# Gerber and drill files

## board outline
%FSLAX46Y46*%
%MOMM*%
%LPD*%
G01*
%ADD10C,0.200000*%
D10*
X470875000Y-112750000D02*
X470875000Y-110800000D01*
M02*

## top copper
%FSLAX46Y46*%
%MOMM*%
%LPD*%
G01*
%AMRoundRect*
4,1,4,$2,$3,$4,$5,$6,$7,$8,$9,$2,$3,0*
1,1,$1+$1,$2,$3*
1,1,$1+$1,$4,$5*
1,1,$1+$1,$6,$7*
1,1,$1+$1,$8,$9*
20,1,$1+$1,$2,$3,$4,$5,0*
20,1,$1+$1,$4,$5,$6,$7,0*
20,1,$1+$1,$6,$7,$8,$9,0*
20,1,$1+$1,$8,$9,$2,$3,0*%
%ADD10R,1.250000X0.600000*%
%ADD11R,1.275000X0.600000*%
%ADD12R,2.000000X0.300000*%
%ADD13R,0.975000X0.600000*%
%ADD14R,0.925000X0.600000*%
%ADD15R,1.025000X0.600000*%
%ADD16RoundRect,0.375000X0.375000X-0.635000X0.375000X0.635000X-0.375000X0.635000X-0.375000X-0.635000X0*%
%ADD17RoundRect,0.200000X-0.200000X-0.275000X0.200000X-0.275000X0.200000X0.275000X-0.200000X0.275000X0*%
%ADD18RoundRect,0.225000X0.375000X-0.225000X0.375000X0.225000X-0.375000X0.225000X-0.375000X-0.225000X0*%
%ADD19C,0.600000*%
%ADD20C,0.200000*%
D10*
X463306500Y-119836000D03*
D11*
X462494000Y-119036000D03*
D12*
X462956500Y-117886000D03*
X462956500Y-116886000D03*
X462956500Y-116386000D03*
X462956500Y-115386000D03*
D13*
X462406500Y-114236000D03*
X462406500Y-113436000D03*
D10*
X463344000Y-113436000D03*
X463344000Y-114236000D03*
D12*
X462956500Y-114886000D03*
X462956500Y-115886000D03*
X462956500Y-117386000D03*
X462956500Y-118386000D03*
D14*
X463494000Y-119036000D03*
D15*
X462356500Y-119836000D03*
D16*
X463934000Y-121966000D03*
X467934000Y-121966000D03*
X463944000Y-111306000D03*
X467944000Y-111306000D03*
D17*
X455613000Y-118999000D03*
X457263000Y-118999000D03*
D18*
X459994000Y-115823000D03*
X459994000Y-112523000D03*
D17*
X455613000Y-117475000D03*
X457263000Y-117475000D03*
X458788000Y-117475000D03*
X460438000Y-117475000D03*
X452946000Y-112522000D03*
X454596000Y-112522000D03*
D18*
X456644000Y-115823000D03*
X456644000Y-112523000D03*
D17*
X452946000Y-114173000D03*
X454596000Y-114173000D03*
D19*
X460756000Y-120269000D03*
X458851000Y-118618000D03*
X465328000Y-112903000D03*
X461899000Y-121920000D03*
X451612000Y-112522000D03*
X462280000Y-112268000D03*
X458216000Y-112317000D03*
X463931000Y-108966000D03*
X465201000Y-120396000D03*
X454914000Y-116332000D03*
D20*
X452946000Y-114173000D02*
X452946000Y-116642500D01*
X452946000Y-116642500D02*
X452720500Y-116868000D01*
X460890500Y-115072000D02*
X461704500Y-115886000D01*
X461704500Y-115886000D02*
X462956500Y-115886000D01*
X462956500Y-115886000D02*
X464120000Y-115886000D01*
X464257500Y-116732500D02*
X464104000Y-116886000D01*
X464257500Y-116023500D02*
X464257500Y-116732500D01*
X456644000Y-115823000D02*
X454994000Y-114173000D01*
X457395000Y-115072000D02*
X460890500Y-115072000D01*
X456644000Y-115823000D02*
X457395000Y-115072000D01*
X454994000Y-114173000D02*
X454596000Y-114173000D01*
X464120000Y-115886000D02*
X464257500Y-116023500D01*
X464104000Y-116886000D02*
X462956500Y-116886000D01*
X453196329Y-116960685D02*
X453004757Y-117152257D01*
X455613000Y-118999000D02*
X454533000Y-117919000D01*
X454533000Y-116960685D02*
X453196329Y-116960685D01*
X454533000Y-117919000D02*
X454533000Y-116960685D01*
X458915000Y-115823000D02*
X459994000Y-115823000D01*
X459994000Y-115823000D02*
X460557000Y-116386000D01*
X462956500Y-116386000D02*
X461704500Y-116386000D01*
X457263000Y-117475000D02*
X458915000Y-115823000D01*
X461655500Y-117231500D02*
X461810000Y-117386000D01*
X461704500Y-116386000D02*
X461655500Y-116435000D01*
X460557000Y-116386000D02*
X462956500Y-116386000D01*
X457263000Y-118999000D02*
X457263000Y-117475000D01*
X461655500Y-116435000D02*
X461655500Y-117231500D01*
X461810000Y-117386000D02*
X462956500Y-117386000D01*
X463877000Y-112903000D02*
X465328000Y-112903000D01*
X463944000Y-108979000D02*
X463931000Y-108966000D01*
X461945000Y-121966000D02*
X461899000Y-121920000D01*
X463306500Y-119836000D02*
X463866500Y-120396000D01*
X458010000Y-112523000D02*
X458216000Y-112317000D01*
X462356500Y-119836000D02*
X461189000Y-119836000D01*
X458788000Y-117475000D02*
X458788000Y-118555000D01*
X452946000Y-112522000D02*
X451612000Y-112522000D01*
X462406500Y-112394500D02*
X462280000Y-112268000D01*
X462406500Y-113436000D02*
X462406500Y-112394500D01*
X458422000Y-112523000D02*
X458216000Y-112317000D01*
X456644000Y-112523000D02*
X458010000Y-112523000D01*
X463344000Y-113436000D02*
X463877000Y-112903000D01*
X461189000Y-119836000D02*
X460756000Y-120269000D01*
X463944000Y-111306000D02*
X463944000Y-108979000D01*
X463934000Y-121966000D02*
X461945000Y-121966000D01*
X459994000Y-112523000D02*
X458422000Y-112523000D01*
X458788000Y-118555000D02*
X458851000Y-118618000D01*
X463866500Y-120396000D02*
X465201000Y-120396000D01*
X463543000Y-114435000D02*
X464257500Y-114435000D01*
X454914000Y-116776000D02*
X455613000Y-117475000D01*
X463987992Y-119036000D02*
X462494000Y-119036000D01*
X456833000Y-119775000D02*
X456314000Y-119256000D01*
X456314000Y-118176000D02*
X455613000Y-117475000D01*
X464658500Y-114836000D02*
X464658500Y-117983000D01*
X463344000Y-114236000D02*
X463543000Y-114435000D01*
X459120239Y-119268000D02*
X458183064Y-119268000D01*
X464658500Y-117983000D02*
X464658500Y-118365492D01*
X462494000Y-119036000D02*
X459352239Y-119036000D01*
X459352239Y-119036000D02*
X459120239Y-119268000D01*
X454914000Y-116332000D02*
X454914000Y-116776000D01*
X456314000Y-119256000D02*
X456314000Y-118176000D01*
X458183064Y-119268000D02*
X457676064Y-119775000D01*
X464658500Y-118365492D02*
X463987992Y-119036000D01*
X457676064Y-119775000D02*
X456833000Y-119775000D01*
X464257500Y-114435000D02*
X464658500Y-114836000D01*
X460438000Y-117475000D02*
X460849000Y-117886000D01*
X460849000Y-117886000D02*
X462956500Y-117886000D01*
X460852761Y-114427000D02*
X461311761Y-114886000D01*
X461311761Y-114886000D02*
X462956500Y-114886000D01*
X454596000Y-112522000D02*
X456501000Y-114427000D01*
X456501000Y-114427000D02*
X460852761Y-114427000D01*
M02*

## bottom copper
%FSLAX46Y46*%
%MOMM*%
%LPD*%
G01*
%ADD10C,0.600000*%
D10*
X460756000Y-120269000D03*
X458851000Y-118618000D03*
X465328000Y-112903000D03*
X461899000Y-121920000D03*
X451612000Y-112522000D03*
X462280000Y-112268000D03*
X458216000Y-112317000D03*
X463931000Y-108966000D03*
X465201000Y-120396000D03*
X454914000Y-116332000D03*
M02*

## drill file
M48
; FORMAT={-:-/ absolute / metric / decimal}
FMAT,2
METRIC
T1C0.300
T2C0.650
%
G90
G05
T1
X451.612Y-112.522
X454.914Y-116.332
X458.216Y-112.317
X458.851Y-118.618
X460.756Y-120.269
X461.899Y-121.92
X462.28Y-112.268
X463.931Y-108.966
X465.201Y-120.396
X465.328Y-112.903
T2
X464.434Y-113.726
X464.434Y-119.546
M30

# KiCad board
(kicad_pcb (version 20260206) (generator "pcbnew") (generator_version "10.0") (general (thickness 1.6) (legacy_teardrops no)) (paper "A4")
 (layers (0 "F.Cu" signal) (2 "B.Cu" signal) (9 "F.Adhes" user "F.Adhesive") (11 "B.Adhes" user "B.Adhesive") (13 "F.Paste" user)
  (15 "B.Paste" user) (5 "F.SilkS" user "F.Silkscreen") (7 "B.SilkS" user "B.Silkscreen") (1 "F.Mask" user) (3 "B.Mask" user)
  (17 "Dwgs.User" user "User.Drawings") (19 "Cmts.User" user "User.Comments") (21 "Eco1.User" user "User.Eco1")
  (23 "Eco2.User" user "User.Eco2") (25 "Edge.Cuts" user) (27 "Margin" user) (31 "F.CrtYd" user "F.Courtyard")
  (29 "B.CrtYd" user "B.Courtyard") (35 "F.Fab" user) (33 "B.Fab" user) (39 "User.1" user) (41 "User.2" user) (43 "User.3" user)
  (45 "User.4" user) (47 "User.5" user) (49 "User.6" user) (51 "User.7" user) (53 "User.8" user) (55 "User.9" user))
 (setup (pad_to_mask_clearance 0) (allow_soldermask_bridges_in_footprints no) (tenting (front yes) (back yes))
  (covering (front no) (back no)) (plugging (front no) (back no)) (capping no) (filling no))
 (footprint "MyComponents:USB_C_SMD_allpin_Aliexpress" (layer "F.Cu") (at 463.944 116.636 90)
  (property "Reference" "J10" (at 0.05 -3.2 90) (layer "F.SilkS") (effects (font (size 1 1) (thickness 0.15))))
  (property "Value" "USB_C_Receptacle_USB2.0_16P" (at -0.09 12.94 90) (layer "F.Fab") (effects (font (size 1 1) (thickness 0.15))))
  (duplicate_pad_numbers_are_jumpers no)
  (pad "" np_thru_hole circle (at -2.91 0.49 90) (size 0.65 0.65) (drill 0.65) (layers "*.Cu" "*.Mask"))
  (pad "" np_thru_hole circle (at 2.91 0.49 90) (size 0.65 0.65) (drill 0.65) (layers "*.Cu" "*.Mask"))
  (pad "A1" smd rect (at -3.2 -0.6375 90) (size 0.6 1.25) (layers "F.Cu" "F.Mask" "F.Paste") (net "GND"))
  (pad "A4" smd rect (at -2.4 -1.45 90) (size 0.6 1.275) (layers "F.Cu" "F.Mask" "F.Paste") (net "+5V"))
  (pad "A5" smd rect (at -1.25 -0.9875 90) (size 0.3 2) (layers "F.Cu" "F.Mask" "F.Paste") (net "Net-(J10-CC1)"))
  (pad "A6" smd rect (at -0.25 -0.9875 90) (size 0.3 2) (layers "F.Cu" "F.Mask" "F.Paste") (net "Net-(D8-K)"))
  (pad "A7" smd rect (at 0.25 -0.9875 270) (size 0.3 2) (layers "F.Cu" "F.Mask" "F.Paste") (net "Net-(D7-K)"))
  (pad "A8" smd rect (at 1.25 -0.9875 270) (size 0.3 2) (layers "F.Cu" "F.Mask" "F.Paste") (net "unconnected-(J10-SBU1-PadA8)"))
  (pad "A9" smd rect (at 2.4 -1.5375 270) (size 0.6 0.975) (layers "F.Cu" "F.Mask" "F.Paste") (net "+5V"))
  (pad "A12" smd rect (at 3.2 -1.5375 270) (size 0.6 0.975) (layers "F.Cu" "F.Mask" "F.Paste") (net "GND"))
  (pad "B1" smd rect (at 3.2 -0.6 270) (size 0.6 1.25) (layers "F.Cu" "F.Mask" "F.Paste") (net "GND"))
  (pad "B4" smd rect (at 2.4 -0.6 270) (size 0.6 1.25) (layers "F.Cu" "F.Mask" "F.Paste") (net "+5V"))
  (pad "B5" smd rect (at 1.75 -0.9875 270) (size 0.3 2) (layers "F.Cu" "F.Mask" "F.Paste") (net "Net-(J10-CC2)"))
  (pad "B6" smd rect (at 0.75 -0.9875 270) (size 0.3 2) (layers "F.Cu" "F.Mask" "F.Paste") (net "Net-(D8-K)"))
  (pad "B7" smd rect (at -0.75 -0.9875 90) (size 0.3 2) (layers "F.Cu" "F.Mask" "F.Paste") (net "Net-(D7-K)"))
  (pad "B8" smd rect (at -1.75 -0.9875 90) (size 0.3 2) (layers "F.Cu" "F.Mask" "F.Paste") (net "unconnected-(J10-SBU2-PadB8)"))
  (pad "B9" smd rect (at -2.4 -0.45 90) (size 0.6 0.925) (layers "F.Cu" "F.Mask" "F.Paste") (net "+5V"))
  (pad "B12" smd rect (at -3.2 -1.5875 90) (size 0.6 1.025) (layers "F.Cu" "F.Mask" "F.Paste") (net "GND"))
  (pad "S1" smd roundrect (at -5.33 -0.01 90) (size 2.02 1.5) (layers "F.Cu" "F.Mask" "F.Paste") (roundrect_rratio 0.25) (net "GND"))
  (pad "S1" smd roundrect (at -5.33 3.99 90) (size 2.02 1.5) (layers "F.Cu" "F.Mask" "F.Paste") (roundrect_rratio 0.25) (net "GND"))
  (pad "S1" smd roundrect (at 5.33 0 90) (size 2.02 1.5) (layers "F.Cu" "F.Mask" "F.Paste") (roundrect_rratio 0.25) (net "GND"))
  (pad "S1" smd roundrect (at 5.33 4 90) (size 2.02 1.5) (layers "F.Cu" "F.Mask" "F.Paste") (roundrect_rratio 0.25) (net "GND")))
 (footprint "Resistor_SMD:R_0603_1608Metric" (layer "F.Cu") (at 456.438 118.999)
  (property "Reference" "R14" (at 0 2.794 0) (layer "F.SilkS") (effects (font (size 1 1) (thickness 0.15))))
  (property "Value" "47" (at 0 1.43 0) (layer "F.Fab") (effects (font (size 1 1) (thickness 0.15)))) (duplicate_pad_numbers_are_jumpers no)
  (pad "1" smd roundrect (at -0.825 0) (size 0.8 0.95) (layers "F.Cu" "F.Mask" "F.Paste") (roundrect_rratio 0.25) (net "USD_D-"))
  (pad "2" smd roundrect (at 0.825 0) (size 0.8 0.95) (layers "F.Cu" "F.Mask" "F.Paste") (roundrect_rratio 0.25) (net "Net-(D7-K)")))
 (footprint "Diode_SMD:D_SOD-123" (layer "F.Cu") (at 459.994 114.173 90)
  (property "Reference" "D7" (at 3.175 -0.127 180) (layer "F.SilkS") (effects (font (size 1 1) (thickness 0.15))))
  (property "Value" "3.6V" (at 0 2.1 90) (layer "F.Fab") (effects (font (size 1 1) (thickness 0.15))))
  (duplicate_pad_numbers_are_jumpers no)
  (pad "1" smd roundrect (at -1.65 0 90) (size 0.9 1.2) (layers "F.Cu" "F.Mask" "F.Paste") (roundrect_rratio 0.25) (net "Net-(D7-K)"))
  (pad "2" smd roundrect (at 1.65 0 90) (size 0.9 1.2) (layers "F.Cu" "F.Mask" "F.Paste") (roundrect_rratio 0.25) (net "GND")))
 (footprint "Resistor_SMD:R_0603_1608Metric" (layer "F.Cu") (at 456.438 117.475)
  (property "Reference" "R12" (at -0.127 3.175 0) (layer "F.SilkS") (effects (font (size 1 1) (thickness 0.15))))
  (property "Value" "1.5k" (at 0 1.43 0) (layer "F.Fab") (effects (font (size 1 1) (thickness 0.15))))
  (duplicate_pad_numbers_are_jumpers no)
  (pad "1" smd roundrect (at -0.825 0) (size 0.8 0.95) (layers "F.Cu" "F.Mask" "F.Paste") (roundrect_rratio 0.25) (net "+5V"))
  (pad "2" smd roundrect (at 0.825 0) (size 0.8 0.95) (layers "F.Cu" "F.Mask" "F.Paste") (roundrect_rratio 0.25) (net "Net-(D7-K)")))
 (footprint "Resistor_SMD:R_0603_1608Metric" (layer "F.Cu") (at 459.613 117.475)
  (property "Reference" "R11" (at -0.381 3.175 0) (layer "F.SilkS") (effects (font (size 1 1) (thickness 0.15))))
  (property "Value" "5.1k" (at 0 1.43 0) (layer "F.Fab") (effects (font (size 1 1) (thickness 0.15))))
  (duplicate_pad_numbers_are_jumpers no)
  (pad "1" smd roundrect (at -0.825 0) (size 0.8 0.95) (layers "F.Cu" "F.Mask" "F.Paste") (roundrect_rratio 0.25) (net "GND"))
  (pad "2" smd roundrect (at 0.825 0) (size 0.8 0.95) (layers "F.Cu" "F.Mask" "F.Paste") (roundrect_rratio 0.25) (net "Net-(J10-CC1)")))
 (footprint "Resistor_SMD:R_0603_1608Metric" (layer "F.Cu") (at 453.771 112.522)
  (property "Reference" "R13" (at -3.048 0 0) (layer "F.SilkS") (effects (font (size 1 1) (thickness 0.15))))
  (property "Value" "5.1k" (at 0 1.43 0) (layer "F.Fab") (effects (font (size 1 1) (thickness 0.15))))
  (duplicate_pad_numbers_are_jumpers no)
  (pad "1" smd roundrect (at -0.825 0) (size 0.8 0.95) (layers "F.Cu" "F.Mask" "F.Paste") (roundrect_rratio 0.25) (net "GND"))
  (pad "2" smd roundrect (at 0.825 0) (size 0.8 0.95) (layers "F.Cu" "F.Mask" "F.Paste") (roundrect_rratio 0.25) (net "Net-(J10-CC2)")))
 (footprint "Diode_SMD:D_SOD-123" (layer "F.Cu") (at 456.644 114.173 90)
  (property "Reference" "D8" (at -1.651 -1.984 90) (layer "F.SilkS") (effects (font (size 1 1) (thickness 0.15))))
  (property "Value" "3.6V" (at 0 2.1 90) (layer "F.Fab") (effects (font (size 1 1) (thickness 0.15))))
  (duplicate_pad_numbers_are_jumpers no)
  (pad "1" smd roundrect (at -1.65 0 90) (size 0.9 1.2) (layers "F.Cu" "F.Mask" "F.Paste") (roundrect_rratio 0.25) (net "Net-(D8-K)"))
  (pad "2" smd roundrect (at 1.65 0 90) (size 0.9 1.2) (layers "F.Cu" "F.Mask" "F.Paste") (roundrect_rratio 0.25) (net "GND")))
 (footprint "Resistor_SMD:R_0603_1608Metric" (layer "F.Cu") (at 453.771 114.173)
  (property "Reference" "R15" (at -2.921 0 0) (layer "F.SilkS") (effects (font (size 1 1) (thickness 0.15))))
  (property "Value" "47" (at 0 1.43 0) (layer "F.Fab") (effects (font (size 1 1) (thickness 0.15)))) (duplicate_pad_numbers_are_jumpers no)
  (pad "1" smd roundrect (at -0.825 0) (size 0.8 0.95) (layers "F.Cu" "F.Mask" "F.Paste") (roundrect_rratio 0.25) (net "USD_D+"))
  (pad "2" smd roundrect (at 0.825 0) (size 0.8 0.95) (layers "F.Cu" "F.Mask" "F.Paste") (roundrect_rratio 0.25) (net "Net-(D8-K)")))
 (gr_line (start 470.875 112.75) (end 470.875 110.8) (stroke (width 0.2) (type default)) (layer "Edge.Cuts"))
 (segment (start 452.946 114.173) (end 452.946 116.6425) (width 0.2) (layer "F.Cu") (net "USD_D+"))
 (segment (start 452.946 116.6425) (end 452.7205 116.868) (width 0.2) (layer "F.Cu") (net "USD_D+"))
 (segment (start 460.8905 115.072) (end 461.7045 115.886) (width 0.2) (layer "F.Cu") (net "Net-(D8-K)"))
 (segment (start 461.7045 115.886) (end 462.9565 115.886) (width 0.2) (layer "F.Cu") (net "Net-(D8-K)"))
 (segment (start 462.9565 115.886) (end 464.12 115.886) (width 0.2) (layer "F.Cu") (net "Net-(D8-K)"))
 (segment (start 464.2575 116.7325) (end 464.104 116.886) (width 0.2) (layer "F.Cu") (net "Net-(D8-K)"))
 (segment (start 464.2575 116.0235) (end 464.2575 116.7325) (width 0.2) (layer "F.Cu") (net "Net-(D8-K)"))
 (segment (start 456.644 115.823) (end 454.994 114.173) (width 0.2) (layer "F.Cu") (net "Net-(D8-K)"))
 (segment (start 457.395 115.072) (end 460.8905 115.072) (width 0.2) (layer "F.Cu") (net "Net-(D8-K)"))
 (segment (start 456.644 115.823) (end 457.395 115.072) (width 0.2) (layer "F.Cu") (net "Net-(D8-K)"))
 (segment (start 454.994 114.173) (end 454.596 114.173) (width 0.2) (layer "F.Cu") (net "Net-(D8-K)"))
 (segment (start 464.12 115.886) (end 464.2575 116.0235) (width 0.2) (layer "F.Cu") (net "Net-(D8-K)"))
 (segment (start 464.104 116.886) (end 462.9565 116.886) (width 0.2) (layer "F.Cu") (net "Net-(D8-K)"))
 (segment (start 453.196329 116.960685) (end 453.004757 117.152257) (width 0.2) (layer "F.Cu") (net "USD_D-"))
 (segment (start 455.613 118.999) (end 454.533 117.919) (width 0.2) (layer "F.Cu") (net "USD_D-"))
 (segment (start 454.533 116.960685) (end 453.196329 116.960685) (width 0.2) (layer "F.Cu") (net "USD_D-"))
 (segment (start 454.533 117.919) (end 454.533 116.960685) (width 0.2) (layer "F.Cu") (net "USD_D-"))
 (segment (start 458.915 115.823) (end 459.994 115.823) (width 0.2) (layer "F.Cu") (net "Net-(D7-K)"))
 (segment (start 459.994 115.823) (end 460.557 116.386) (width 0.2) (layer "F.Cu") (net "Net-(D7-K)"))
 (segment (start 462.9565 116.386) (end 461.7045 116.386) (width 0.2) (layer "F.Cu") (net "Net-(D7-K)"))
 (segment (start 457.263 117.475) (end 458.915 115.823) (width 0.2) (layer "F.Cu") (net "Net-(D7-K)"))
 (segment (start 461.6555 117.2315) (end 461.81 117.386) (width 0.2) (layer "F.Cu") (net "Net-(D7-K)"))
 (segment (start 461.7045 116.386) (end 461.6555 116.435) (width 0.2) (layer "F.Cu") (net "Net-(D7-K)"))
 (segment (start 460.557 116.386) (end 462.9565 116.386) (width 0.2) (layer "F.Cu") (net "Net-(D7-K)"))
 (segment (start 457.263 118.999) (end 457.263 117.475) (width 0.2) (layer "F.Cu") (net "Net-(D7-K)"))
 (segment (start 461.6555 116.435) (end 461.6555 117.2315) (width 0.2) (layer "F.Cu") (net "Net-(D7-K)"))
 (segment (start 461.81 117.386) (end 462.9565 117.386) (width 0.2) (layer "F.Cu") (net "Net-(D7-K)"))
 (segment (start 463.877 112.903) (end 465.328 112.903) (width 0.2) (layer "F.Cu") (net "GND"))
 (segment (start 463.944 108.979) (end 463.931 108.966) (width 0.2) (layer "F.Cu") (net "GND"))
 (segment (start 461.945 121.966) (end 461.899 121.92) (width 0.2) (layer "F.Cu") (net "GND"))
 (segment (start 463.3065 119.836) (end 463.8665 120.396) (width 0.2) (layer "F.Cu") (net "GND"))
 (segment (start 458.01 112.523) (end 458.216 112.317) (width 0.2) (layer "F.Cu") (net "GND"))
 (segment (start 462.3565 119.836) (end 461.189 119.836) (width 0.2) (layer "F.Cu") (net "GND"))
 (segment (start 458.788 117.475) (end 458.788 118.555) (width 0.2) (layer "F.Cu") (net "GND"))
 (segment (start 452.946 112.522) (end 451.612 112.522) (width 0.2) (layer "F.Cu") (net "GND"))
 (segment (start 462.4065 112.3945) (end 462.28 112.268) (width 0.2) (layer "F.Cu") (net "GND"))
 (segment (start 462.4065 113.436) (end 462.4065 112.3945) (width 0.2) (layer "F.Cu") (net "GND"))
 (segment (start 458.422 112.523) (end 458.216 112.317) (width 0.2) (layer "F.Cu") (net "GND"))
 (segment (start 456.644 112.523) (end 458.01 112.523) (width 0.2) (layer "F.Cu") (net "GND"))
 (segment (start 463.344 113.436) (end 463.877 112.903) (width 0.2) (layer "F.Cu") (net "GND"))
 (segment (start 461.189 119.836) (end 460.756 120.269) (width 0.2) (layer "F.Cu") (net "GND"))
 (segment (start 463.944 111.306) (end 463.944 108.979) (width 0.2) (layer "F.Cu") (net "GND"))
 (segment (start 463.934 121.966) (end 461.945 121.966) (width 0.2) (layer "F.Cu") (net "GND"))
 (segment (start 459.994 112.523) (end 458.422 112.523) (width 0.2) (layer "F.Cu") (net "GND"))
 (segment (start 458.788 118.555) (end 458.851 118.618) (width 0.2) (layer "F.Cu") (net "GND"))
 (segment (start 463.8665 120.396) (end 465.201 120.396) (width 0.2) (layer "F.Cu") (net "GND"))
 (via (at 460.756 120.269) (size 0.6) (drill 0.3) (layers "F.Cu" "B.Cu") (capping no) (covering (front no) (back no))
  (plugging (front no) (back no)) (filling no) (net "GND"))
 (via (at 458.851 118.618) (size 0.6) (drill 0.3) (layers "F.Cu" "B.Cu") (capping no) (covering (front no) (back no))
  (plugging (front no) (back no)) (filling no) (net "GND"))
 (via (at 465.328 112.903) (size 0.6) (drill 0.3) (layers "F.Cu" "B.Cu") (capping no) (covering (front no) (back no))
  (plugging (front no) (back no)) (filling no) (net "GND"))
 (via (at 461.899 121.92) (size 0.6) (drill 0.3) (layers "F.Cu" "B.Cu") (capping no) (covering (front no) (back no))
  (plugging (front no) (back no)) (filling no) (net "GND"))
 (via (at 451.612 112.522) (size 0.6) (drill 0.3) (layers "F.Cu" "B.Cu") (capping no) (covering (front no) (back no))
  (plugging (front no) (back no)) (filling no) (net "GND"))
 (via (at 462.28 112.268) (size 0.6) (drill 0.3) (layers "F.Cu" "B.Cu") (capping no) (covering (front no) (back no))
  (plugging (front no) (back no)) (filling no) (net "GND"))
 (via (at 458.216 112.317) (size 0.6) (drill 0.3) (layers "F.Cu" "B.Cu") (capping no) (covering (front no) (back no))
  (plugging (front no) (back no)) (filling no) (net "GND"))
 (via (at 463.931 108.966) (size 0.6) (drill 0.3) (layers "F.Cu" "B.Cu") (capping no) (covering (front no) (back no))
  (plugging (front no) (back no)) (filling no) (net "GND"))
 (via (at 465.201 120.396) (size 0.6) (drill 0.3) (layers "F.Cu" "B.Cu") (capping no) (covering (front no) (back no))
  (plugging (front no) (back no)) (filling no) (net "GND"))
 (segment (start 463.543 114.435) (end 464.2575 114.435) (width 0.2) (layer "F.Cu") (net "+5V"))
 (segment (start 454.914 116.776) (end 455.613 117.475) (width 0.2) (layer "F.Cu") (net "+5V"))
 (segment (start 463.987992 119.036) (end 462.494 119.036) (width 0.2) (layer "F.Cu") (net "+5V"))
 (segment (start 456.833 119.775) (end 456.314 119.256) (width 0.2) (layer "F.Cu") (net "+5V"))
 (segment (start 456.314 118.176) (end 455.613 117.475) (width 0.2) (layer "F.Cu") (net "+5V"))
 (segment (start 464.6585 114.836) (end 464.6585 117.983) (width 0.2) (layer "F.Cu") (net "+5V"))
 (segment (start 463.344 114.236) (end 463.543 114.435) (width 0.2) (layer "F.Cu") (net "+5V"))
 (segment (start 459.120239 119.268) (end 458.183064 119.268) (width 0.2) (layer "F.Cu") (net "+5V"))
 (segment (start 464.6585 117.983) (end 464.6585 118.365492) (width 0.2) (layer "F.Cu") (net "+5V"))
 (segment (start 462.494 119.036) (end 459.352239 119.036) (width 0.2) (layer "F.Cu") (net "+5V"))
 (segment (start 459.352239 119.036) (end 459.120239 119.268) (width 0.2) (layer "F.Cu") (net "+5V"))
 (segment (start 454.914 116.332) (end 454.914 116.776) (width 0.2) (layer "F.Cu") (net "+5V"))
 (segment (start 456.314 119.256) (end 456.314 118.176) (width 0.2) (layer "F.Cu") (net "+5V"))
 (segment (start 458.183064 119.268) (end 457.676064 119.775) (width 0.2) (layer "F.Cu") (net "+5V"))
 (segment (start 464.6585 118.365492) (end 463.987992 119.036) (width 0.2) (layer "F.Cu") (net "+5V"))
 (segment (start 457.676064 119.775) (end 456.833 119.775) (width 0.2) (layer "F.Cu") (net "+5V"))
 (segment (start 464.2575 114.435) (end 464.6585 114.836) (width 0.2) (layer "F.Cu") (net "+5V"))
 (via (at 454.914 116.332) (size 0.6) (drill 0.3) (layers "F.Cu" "B.Cu") (capping no) (covering (front no) (back no))
  (plugging (front no) (back no)) (filling no) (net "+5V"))
 (segment (start 460.438 117.475) (end 460.849 117.886) (width 0.2) (layer "F.Cu") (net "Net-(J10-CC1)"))
 (segment (start 460.849 117.886) (end 462.9565 117.886) (width 0.2) (layer "F.Cu") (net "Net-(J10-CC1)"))
 (segment (start 460.852761 114.427) (end 461.311761 114.886) (width 0.2) (layer "F.Cu") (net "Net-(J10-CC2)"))
 (segment (start 461.311761 114.886) (end 462.9565 114.886) (width 0.2) (layer "F.Cu") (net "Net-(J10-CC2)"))
 (segment (start 454.596 112.522) (end 456.501 114.427) (width 0.2) (layer "F.Cu") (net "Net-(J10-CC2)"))
 (segment (start 456.501 114.427) (end 460.852761 114.427) (width 0.2) (layer "F.Cu") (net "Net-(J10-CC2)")))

